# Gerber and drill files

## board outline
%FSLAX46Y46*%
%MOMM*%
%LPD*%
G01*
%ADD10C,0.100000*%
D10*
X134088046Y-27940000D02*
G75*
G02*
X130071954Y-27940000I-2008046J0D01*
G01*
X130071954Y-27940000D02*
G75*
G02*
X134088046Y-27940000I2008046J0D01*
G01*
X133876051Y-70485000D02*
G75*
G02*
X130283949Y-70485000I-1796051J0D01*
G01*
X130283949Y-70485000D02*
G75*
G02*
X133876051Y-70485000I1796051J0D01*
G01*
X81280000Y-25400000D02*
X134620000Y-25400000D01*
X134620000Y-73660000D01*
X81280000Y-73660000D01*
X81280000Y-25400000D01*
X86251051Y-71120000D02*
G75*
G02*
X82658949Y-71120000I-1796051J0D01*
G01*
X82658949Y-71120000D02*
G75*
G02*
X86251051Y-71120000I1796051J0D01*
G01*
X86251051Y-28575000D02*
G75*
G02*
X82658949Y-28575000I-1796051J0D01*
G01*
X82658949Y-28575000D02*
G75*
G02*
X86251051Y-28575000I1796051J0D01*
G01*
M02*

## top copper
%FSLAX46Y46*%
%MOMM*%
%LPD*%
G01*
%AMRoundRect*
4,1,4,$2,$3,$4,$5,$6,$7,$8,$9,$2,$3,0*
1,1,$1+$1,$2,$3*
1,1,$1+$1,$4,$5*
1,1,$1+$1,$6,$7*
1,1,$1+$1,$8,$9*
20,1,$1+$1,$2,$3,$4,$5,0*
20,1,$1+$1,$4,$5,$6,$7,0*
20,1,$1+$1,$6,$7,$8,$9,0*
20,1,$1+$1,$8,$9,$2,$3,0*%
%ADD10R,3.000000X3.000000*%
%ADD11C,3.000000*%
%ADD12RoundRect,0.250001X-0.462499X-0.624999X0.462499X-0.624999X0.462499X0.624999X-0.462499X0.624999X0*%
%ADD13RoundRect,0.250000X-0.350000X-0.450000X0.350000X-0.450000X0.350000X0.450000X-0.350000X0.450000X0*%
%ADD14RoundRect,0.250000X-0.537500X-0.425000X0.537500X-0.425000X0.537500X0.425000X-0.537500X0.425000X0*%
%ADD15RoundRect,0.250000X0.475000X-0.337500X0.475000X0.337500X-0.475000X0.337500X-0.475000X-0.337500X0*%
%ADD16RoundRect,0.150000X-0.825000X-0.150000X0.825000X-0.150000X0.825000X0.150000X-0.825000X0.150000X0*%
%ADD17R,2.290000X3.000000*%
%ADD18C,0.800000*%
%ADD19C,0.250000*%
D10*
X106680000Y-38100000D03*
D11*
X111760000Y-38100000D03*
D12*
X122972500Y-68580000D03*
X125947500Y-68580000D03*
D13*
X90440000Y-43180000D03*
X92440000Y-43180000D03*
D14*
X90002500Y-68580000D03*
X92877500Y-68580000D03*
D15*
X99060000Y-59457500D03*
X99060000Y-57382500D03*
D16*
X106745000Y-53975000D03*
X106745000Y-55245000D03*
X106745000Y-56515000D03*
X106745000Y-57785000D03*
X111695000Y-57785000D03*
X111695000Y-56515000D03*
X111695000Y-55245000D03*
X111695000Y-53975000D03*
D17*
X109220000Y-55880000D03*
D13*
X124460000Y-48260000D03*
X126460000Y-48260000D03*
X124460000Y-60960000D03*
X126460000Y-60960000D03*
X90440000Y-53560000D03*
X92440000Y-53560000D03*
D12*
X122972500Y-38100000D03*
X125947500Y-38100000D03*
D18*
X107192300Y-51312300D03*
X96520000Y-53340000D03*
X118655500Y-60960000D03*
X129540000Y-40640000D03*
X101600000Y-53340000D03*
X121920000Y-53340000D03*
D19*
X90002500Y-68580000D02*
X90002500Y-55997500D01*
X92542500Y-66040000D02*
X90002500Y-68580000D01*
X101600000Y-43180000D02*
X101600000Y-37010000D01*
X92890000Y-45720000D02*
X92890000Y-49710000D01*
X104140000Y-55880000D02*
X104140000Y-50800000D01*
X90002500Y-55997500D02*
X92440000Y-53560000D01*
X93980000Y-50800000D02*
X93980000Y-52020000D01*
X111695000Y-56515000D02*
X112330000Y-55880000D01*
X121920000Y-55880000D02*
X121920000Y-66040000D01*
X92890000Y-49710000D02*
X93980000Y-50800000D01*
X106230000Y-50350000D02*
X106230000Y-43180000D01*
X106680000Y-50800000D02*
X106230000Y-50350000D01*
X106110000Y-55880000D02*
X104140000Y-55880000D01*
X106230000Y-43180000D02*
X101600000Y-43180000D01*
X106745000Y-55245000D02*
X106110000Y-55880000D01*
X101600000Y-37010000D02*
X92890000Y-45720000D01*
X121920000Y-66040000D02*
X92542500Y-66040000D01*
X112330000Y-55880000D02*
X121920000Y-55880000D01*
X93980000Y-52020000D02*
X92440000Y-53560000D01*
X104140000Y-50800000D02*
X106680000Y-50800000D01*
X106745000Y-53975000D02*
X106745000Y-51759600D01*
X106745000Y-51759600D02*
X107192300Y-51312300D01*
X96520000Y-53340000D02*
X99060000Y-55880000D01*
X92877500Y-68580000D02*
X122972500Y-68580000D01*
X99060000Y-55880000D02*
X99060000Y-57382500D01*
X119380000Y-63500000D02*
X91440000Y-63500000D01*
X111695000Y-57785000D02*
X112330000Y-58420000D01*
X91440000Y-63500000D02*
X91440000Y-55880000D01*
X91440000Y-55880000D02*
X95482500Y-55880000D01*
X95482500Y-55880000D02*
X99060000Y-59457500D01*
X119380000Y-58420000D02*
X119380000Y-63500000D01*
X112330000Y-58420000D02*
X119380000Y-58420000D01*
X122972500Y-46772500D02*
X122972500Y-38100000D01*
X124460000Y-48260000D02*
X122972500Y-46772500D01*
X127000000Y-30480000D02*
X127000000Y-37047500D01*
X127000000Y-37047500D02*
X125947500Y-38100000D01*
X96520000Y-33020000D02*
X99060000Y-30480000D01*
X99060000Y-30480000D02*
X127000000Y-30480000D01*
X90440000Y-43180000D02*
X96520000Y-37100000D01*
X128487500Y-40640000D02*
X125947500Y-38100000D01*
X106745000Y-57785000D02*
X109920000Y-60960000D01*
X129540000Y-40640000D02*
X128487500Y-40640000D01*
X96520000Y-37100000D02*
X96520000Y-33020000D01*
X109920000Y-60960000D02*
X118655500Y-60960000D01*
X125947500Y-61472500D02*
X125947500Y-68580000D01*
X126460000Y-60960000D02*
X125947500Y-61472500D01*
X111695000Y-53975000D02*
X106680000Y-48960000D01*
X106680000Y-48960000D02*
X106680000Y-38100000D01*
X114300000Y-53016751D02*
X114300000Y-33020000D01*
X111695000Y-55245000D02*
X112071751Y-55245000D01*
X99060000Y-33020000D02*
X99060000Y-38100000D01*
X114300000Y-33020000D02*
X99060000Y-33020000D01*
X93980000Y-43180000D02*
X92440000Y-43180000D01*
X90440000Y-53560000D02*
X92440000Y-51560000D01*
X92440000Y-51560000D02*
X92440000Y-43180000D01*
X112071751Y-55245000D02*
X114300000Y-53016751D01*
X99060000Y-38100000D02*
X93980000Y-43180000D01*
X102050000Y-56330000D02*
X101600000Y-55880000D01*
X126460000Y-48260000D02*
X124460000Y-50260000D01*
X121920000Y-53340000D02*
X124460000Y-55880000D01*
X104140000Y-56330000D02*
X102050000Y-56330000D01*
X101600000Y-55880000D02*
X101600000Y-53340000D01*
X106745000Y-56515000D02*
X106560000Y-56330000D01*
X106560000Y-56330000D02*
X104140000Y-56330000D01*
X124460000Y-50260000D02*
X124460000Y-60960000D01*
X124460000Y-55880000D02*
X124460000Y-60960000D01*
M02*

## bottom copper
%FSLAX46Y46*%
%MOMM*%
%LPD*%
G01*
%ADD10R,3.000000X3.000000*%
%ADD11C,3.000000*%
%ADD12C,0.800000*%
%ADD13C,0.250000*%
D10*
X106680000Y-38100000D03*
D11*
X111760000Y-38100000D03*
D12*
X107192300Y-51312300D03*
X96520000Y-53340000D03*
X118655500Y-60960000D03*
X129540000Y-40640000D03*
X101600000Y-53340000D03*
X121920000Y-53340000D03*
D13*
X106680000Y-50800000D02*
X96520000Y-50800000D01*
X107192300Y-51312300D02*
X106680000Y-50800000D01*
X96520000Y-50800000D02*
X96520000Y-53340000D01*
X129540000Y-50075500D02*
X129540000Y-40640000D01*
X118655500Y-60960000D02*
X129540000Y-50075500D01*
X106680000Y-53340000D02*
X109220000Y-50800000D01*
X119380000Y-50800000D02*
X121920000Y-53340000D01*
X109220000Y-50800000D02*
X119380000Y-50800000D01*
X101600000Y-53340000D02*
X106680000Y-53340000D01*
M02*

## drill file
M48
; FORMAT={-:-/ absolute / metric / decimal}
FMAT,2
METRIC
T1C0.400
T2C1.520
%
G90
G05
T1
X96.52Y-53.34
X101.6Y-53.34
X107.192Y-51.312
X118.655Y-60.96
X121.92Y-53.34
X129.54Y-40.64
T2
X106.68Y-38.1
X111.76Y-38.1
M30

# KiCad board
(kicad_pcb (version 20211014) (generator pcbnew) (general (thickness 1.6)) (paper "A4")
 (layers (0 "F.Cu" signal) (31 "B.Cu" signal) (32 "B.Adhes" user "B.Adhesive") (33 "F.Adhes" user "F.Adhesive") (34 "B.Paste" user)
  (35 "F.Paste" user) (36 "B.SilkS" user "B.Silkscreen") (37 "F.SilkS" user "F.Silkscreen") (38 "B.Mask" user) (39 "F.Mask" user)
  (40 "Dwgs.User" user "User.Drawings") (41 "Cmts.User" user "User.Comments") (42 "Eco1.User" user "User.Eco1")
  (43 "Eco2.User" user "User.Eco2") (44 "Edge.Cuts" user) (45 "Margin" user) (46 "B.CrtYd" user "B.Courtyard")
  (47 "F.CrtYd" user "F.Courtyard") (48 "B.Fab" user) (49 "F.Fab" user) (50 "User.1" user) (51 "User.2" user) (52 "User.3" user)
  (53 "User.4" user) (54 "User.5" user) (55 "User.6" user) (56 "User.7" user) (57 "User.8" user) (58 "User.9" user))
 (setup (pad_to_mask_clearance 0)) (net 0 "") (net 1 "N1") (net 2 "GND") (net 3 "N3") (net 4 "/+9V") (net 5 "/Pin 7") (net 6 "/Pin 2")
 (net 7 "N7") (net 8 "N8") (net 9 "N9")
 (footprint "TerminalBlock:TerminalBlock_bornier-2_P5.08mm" (layer "F.Cu") (at 106.68 38.1)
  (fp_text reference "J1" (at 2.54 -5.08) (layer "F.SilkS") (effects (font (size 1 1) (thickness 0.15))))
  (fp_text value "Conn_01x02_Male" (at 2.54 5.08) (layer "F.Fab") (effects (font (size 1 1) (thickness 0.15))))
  (pad "1" thru_hole rect (at 0 0) (size 3 3) (drill 1.52) (layers *.Cu *.Mask) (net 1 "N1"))
  (pad "2" thru_hole circle (at 5.08 0) (size 3 3) (drill 1.52) (layers *.Cu *.Mask) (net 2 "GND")))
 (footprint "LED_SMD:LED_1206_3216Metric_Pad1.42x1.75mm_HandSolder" (layer "F.Cu") (at 124.46 68.58)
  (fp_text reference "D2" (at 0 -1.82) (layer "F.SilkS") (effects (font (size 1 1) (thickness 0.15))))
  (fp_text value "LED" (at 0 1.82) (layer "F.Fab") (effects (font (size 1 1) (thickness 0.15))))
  (pad "1" smd roundrect (at -1.4875 0) (size 1.425 1.75) (layers "F.Cu" "F.Paste" "F.Mask") (roundrect_rratio 0.175439) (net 2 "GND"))
  (pad "2" smd roundrect (at 1.4875 0) (size 1.425 1.75) (layers "F.Cu" "F.Paste" "F.Mask") (roundrect_rratio 0.175439) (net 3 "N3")))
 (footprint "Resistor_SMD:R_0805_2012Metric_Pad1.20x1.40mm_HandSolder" (layer "F.Cu") (at 91.44 43.18)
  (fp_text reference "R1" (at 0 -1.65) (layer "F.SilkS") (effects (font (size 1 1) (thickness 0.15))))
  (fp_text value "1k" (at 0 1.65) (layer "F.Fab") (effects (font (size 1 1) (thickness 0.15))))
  (pad "1" smd roundrect (at -1 0) (size 1.2 1.4) (layers "F.Cu" "F.Paste" "F.Mask") (roundrect_rratio 0.208333) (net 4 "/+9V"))
  (pad "2" smd roundrect (at 1 0) (size 1.2 1.4) (layers "F.Cu" "F.Paste" "F.Mask") (roundrect_rratio 0.208333) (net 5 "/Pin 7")))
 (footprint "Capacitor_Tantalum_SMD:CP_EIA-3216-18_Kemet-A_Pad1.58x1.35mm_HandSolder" (layer "F.Cu") (at 91.44 68.58)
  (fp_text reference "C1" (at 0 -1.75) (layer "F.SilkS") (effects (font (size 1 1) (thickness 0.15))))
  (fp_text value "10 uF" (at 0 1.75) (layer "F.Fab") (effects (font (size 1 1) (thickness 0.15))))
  (pad "1" smd roundrect (at -1.4375 0) (size 1.575 1.35) (layers "F.Cu" "F.Paste" "F.Mask") (roundrect_rratio 0.185185) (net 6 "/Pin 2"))
  (pad "2" smd roundrect (at 1.4375 0) (size 1.575 1.35) (layers "F.Cu" "F.Paste" "F.Mask") (roundrect_rratio 0.185185) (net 2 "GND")))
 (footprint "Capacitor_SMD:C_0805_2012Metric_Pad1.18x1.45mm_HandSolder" (layer "F.Cu") (at 99.06 58.42 90)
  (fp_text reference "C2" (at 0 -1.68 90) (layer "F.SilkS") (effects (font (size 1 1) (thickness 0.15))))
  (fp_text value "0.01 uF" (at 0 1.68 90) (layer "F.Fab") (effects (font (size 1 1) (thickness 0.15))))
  (pad "1" smd roundrect (at -1.0375 0 90) (size 1.175 1.45) (layers "F.Cu" "F.Paste" "F.Mask") (roundrect_rratio 0.212766) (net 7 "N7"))
  (pad "2" smd roundrect (at 1.0375 0 90) (size 1.175 1.45) (layers "F.Cu" "F.Paste" "F.Mask") (roundrect_rratio 0.212766) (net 2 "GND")))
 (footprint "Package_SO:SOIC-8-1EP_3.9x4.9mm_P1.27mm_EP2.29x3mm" (layer "F.Cu") (at 109.22 55.88)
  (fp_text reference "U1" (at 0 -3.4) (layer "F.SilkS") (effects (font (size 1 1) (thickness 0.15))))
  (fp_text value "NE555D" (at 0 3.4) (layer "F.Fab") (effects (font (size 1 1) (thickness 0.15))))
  (pad "" smd roundrect (at -0.57 0.75) (size 0.92 1.21) (layers "F.Paste") (roundrect_rratio 0.25))
  (pad "" smd roundrect (at -0.57 -0.75) (size 0.92 1.21) (layers "F.Paste") (roundrect_rratio 0.25))
  (pad "" smd roundrect (at 0.57 -0.75) (size 0.92 1.21) (layers "F.Paste") (roundrect_rratio 0.25))
  (pad "" smd roundrect (at 0.57 0.75) (size 0.92 1.21) (layers "F.Paste") (roundrect_rratio 0.25))
  (pad "1" smd roundrect (at -2.475 -1.905) (size 1.95 0.6) (layers "F.Cu" "F.Paste" "F.Mask") (roundrect_rratio 0.25) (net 2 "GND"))
  (pad "2" smd roundrect (at -2.475 -0.635) (size 1.95 0.6) (layers "F.Cu" "F.Paste" "F.Mask") (roundrect_rratio 0.25) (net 6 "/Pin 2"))
  (pad "3" smd roundrect (at -2.475 0.635) (size 1.95 0.6) (layers "F.Cu" "F.Paste" "F.Mask") (roundrect_rratio 0.25) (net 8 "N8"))
  (pad "4" smd roundrect (at -2.475 1.905) (size 1.95 0.6) (layers "F.Cu" "F.Paste" "F.Mask") (roundrect_rratio 0.25) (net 4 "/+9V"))
  (pad "5" smd roundrect (at 2.475 1.905) (size 1.95 0.6) (layers "F.Cu" "F.Paste" "F.Mask") (roundrect_rratio 0.25) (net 7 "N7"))
  (pad "6" smd roundrect (at 2.475 0.635) (size 1.95 0.6) (layers "F.Cu" "F.Paste" "F.Mask") (roundrect_rratio 0.25) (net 6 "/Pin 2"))
  (pad "7" smd roundrect (at 2.475 -0.635) (size 1.95 0.6) (layers "F.Cu" "F.Paste" "F.Mask") (roundrect_rratio 0.25) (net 5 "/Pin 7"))
  (pad "8" smd roundrect (at 2.475 -1.905) (size 1.95 0.6) (layers "F.Cu" "F.Paste" "F.Mask") (roundrect_rratio 0.25) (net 1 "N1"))
  (pad "9" smd rect (at 0 0) (size 2.29 3) (layers "F.Cu" "F.Mask")))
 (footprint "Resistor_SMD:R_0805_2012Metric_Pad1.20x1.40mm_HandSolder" (layer "F.Cu") (at 125.46 48.26)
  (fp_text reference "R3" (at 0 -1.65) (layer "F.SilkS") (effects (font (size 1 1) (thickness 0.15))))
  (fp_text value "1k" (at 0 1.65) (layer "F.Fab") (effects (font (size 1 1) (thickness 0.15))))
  (pad "1" smd roundrect (at -1 0) (size 1.2 1.4) (layers "F.Cu" "F.Paste" "F.Mask") (roundrect_rratio 0.208333) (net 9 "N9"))
  (pad "2" smd roundrect (at 1 0) (size 1.2 1.4) (layers "F.Cu" "F.Paste" "F.Mask") (roundrect_rratio 0.208333) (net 8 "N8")))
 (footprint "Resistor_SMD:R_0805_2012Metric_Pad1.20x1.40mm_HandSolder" (layer "F.Cu") (at 125.46 60.96)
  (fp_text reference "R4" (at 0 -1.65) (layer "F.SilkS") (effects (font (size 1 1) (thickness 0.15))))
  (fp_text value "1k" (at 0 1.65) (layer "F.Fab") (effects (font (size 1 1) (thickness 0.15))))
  (pad "1" smd roundrect (at -1 0) (size 1.2 1.4) (layers "F.Cu" "F.Paste" "F.Mask") (roundrect_rratio 0.208333) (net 8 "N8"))
  (pad "2" smd roundrect (at 1 0) (size 1.2 1.4) (layers "F.Cu" "F.Paste" "F.Mask") (roundrect_rratio 0.208333) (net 3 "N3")))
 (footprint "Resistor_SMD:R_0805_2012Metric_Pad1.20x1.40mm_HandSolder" (layer "F.Cu") (at 91.44 53.56)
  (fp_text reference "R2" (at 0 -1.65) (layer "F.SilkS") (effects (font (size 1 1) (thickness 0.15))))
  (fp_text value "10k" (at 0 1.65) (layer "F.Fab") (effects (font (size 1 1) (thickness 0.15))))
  (pad "1" smd roundrect (at -1 0) (size 1.2 1.4) (layers "F.Cu" "F.Paste" "F.Mask") (roundrect_rratio 0.208333) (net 5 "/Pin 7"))
  (pad "2" smd roundrect (at 1 0) (size 1.2 1.4) (layers "F.Cu" "F.Paste" "F.Mask") (roundrect_rratio 0.208333) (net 6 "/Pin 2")))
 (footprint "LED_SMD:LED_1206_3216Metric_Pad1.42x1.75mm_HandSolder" (layer "F.Cu") (at 124.46 38.1)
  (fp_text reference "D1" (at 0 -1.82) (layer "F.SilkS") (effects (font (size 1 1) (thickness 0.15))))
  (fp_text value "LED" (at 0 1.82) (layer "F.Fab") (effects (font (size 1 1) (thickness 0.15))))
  (pad "1" smd roundrect (at -1.4875 0) (size 1.425 1.75) (layers "F.Cu" "F.Paste" "F.Mask") (roundrect_rratio 0.175439) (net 9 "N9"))
  (pad "2" smd roundrect (at 1.4875 0) (size 1.425 1.75) (layers "F.Cu" "F.Paste" "F.Mask") (roundrect_rratio 0.175439) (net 4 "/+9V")))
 (gr_circle (center 132.08 27.94) (end 130.175 28.575) (layer "Edge.Cuts") (width 0.1) (fill none))
 (gr_circle (center 132.08 70.485) (end 130.81 69.215) (layer "Edge.Cuts") (width 0.1) (fill none))
 (gr_rect (start 81.28 25.4) (end 134.62 73.66) (layer "Edge.Cuts") (width 0.1) (fill none))
 (gr_circle (center 84.455 71.12) (end 85.725 69.85) (layer "Edge.Cuts") (width 0.1) (fill none))
 (gr_circle (center 84.455 28.575) (end 85.725 29.845) (layer "Edge.Cuts") (width 0.1) (fill none))
 (segment (start 90.0025 68.58) (end 90.0025 55.9975) (width 0.25) (layer "F.Cu") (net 6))
 (segment (start 92.5425 66.04) (end 90.0025 68.58) (width 0.25) (layer "F.Cu") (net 6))
 (segment (start 101.6 43.18) (end 101.6 37.01) (width 0.25) (layer "F.Cu") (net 6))
 (segment (start 92.89 45.72) (end 92.89 49.71) (width 0.25) (layer "F.Cu") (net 6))
 (segment (start 104.14 55.88) (end 104.14 50.8) (width 0.25) (layer "F.Cu") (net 6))
 (segment (start 90.0025 55.9975) (end 92.44 53.56) (width 0.25) (layer "F.Cu") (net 6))
 (segment (start 93.98 50.8) (end 93.98 52.02) (width 0.25) (layer "F.Cu") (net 6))
 (segment (start 111.695 56.515) (end 112.33 55.88) (width 0.25) (layer "F.Cu") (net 6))
 (segment (start 121.92 55.88) (end 121.92 66.04) (width 0.25) (layer "F.Cu") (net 6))
 (segment (start 92.89 49.71) (end 93.98 50.8) (width 0.25) (layer "F.Cu") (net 6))
 (segment (start 106.23 50.35) (end 106.23 43.18) (width 0.25) (layer "F.Cu") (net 6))
 (segment (start 106.68 50.8) (end 106.23 50.35) (width 0.25) (layer "F.Cu") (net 6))
 (segment (start 106.11 55.88) (end 104.14 55.88) (width 0.25) (layer "F.Cu") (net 6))
 (segment (start 106.23 43.18) (end 101.6 43.18) (width 0.25) (layer "F.Cu") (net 6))
 (segment (start 106.745 55.245) (end 106.11 55.88) (width 0.25) (layer "F.Cu") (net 6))
 (segment (start 101.6 37.01) (end 92.89 45.72) (width 0.25) (layer "F.Cu") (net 6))
 (segment (start 121.92 66.04) (end 92.5425 66.04) (width 0.25) (layer "F.Cu") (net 6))
 (segment (start 112.33 55.88) (end 121.92 55.88) (width 0.25) (layer "F.Cu") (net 6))
 (segment (start 93.98 52.02) (end 92.44 53.56) (width 0.25) (layer "F.Cu") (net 6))
 (segment (start 104.14 50.8) (end 106.68 50.8) (width 0.25) (layer "F.Cu") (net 6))
 (segment (start 106.745 53.975) (end 106.745 51.7596) (width 0.25) (layer "F.Cu") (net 2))
 (segment (start 106.745 51.7596) (end 107.1923 51.3123) (width 0.25) (layer "F.Cu") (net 2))
 (segment (start 96.52 53.34) (end 99.06 55.88) (width 0.25) (layer "F.Cu") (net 2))
 (segment (start 92.8775 68.58) (end 122.9725 68.58) (width 0.25) (layer "F.Cu") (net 2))
 (segment (start 99.06 55.88) (end 99.06 57.3825) (width 0.25) (layer "F.Cu") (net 2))
 (via (at 107.1923 51.3123) (size 0.8) (drill 0.4) (layers "F.Cu" "B.Cu") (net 2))
 (via (at 96.52 53.34) (size 0.8) (drill 0.4) (layers "F.Cu" "B.Cu") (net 2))
 (segment (start 106.68 50.8) (end 96.52 50.8) (width 0.25) (layer "B.Cu") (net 2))
 (segment (start 107.1923 51.3123) (end 106.68 50.8) (width 0.25) (layer "B.Cu") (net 2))
 (segment (start 96.52 50.8) (end 96.52 53.34) (width 0.25) (layer "B.Cu") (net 2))
 (segment (start 119.38 63.5) (end 91.44 63.5) (width 0.25) (layer "F.Cu") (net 7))
 (segment (start 111.695 57.785) (end 112.33 58.42) (width 0.25) (layer "F.Cu") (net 7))
 (segment (start 91.44 63.5) (end 91.44 55.88) (width 0.25) (layer "F.Cu") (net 7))
 (segment (start 91.44 55.88) (end 95.4825 55.88) (width 0.25) (layer "F.Cu") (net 7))
 (segment (start 95.4825 55.88) (end 99.06 59.4575) (width 0.25) (layer "F.Cu") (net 7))
 (segment (start 119.38 58.42) (end 119.38 63.5) (width 0.25) (layer "F.Cu") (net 7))
 (segment (start 112.33 58.42) (end 119.38 58.42) (width 0.25) (layer "F.Cu") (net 7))
 (segment (start 122.9725 46.7725) (end 122.9725 38.1) (width 0.25) (layer "F.Cu") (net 9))
 (segment (start 124.46 48.26) (end 122.9725 46.7725) (width 0.25) (layer "F.Cu") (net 9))
 (segment (start 127 30.48) (end 127 37.0475) (width 0.25) (layer "F.Cu") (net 4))
 (segment (start 127 37.0475) (end 125.9475 38.1) (width 0.25) (layer "F.Cu") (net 4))
 (segment (start 96.52 33.02) (end 99.06 30.48) (width 0.25) (layer "F.Cu") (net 4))
 (segment (start 99.06 30.48) (end 127 30.48) (width 0.25) (layer "F.Cu") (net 4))
 (segment (start 90.44 43.18) (end 96.52 37.1) (width 0.25) (layer "F.Cu") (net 4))
 (segment (start 128.4875 40.64) (end 125.9475 38.1) (width 0.25) (layer "F.Cu") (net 4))
 (segment (start 106.745 57.785) (end 109.92 60.96) (width 0.25) (layer "F.Cu") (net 4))
 (segment (start 129.54 40.64) (end 128.4875 40.64) (width 0.25) (layer "F.Cu") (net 4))
 (segment (start 96.52 37.1) (end 96.52 33.02) (width 0.25) (layer "F.Cu") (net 4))
 (segment (start 109.92 60.96) (end 118.6555 60.96) (width 0.25) (layer "F.Cu") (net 4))
 (via (at 118.6555 60.96) (size 0.8) (drill 0.4) (layers "F.Cu" "B.Cu") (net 4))
 (via (at 129.54 40.64) (size 0.8) (drill 0.4) (layers "F.Cu" "B.Cu") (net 4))
 (segment (start 129.54 50.0755) (end 129.54 40.64) (width 0.25) (layer "B.Cu") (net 4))
 (segment (start 118.6555 60.96) (end 129.54 50.0755) (width 0.25) (layer "B.Cu") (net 4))
 (segment (start 125.9475 61.4725) (end 125.9475 68.58) (width 0.25) (layer "F.Cu") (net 3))
 (segment (start 126.46 60.96) (end 125.9475 61.4725) (width 0.25) (layer "F.Cu") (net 3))
 (segment (start 111.695 53.975) (end 106.68 48.96) (width 0.25) (layer "F.Cu") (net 1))
 (segment (start 106.68 48.96) (end 106.68 38.1) (width 0.25) (layer "F.Cu") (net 1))
 (segment (start 114.3 53.016751) (end 114.3 33.02) (width 0.25) (layer "F.Cu") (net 5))
 (segment (start 111.695 55.245) (end 112.071751 55.245) (width 0.25) (layer "F.Cu") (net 5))
 (segment (start 99.06 33.02) (end 99.06 38.1) (width 0.25) (layer "F.Cu") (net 5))
 (segment (start 114.3 33.02) (end 99.06 33.02) (width 0.25) (layer "F.Cu") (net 5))
 (segment (start 93.98 43.18) (end 92.44 43.18) (width 0.25) (layer "F.Cu") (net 5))
 (segment (start 90.44 53.56) (end 92.44 51.56) (width 0.25) (layer "F.Cu") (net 5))
 (segment (start 92.44 51.56) (end 92.44 43.18) (width 0.25) (layer "F.Cu") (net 5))
 (segment (start 112.071751 55.245) (end 114.3 53.016751) (width 0.25) (layer "F.Cu") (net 5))
 (segment (start 99.06 38.1) (end 93.98 43.18) (width 0.25) (layer "F.Cu") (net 5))
 (segment (start 102.05 56.33) (end 101.6 55.88) (width 0.25) (layer "F.Cu") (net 8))
 (segment (start 126.46 48.26) (end 124.46 50.26) (width 0.25) (layer "F.Cu") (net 8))
 (segment (start 121.92 53.34) (end 124.46 55.88) (width 0.25) (layer "F.Cu") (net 8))
 (segment (start 104.14 56.33) (end 102.05 56.33) (width 0.25) (layer "F.Cu") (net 8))
 (segment (start 101.6 55.88) (end 101.6 53.34) (width 0.25) (layer "F.Cu") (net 8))
 (segment (start 106.745 56.515) (end 106.56 56.33) (width 0.25) (layer "F.Cu") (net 8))
 (segment (start 106.56 56.33) (end 104.14 56.33) (width 0.25) (layer "F.Cu") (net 8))
 (segment (start 124.46 50.26) (end 124.46 60.96) (width 0.25) (layer "F.Cu") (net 8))
 (segment (start 124.46 55.88) (end 124.46 60.96) (width 0.25) (layer "F.Cu") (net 8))
 (via (at 101.6 53.34) (size 0.8) (drill 0.4) (layers "F.Cu" "B.Cu") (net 8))
 (via (at 121.92 53.34) (size 0.8) (drill 0.4) (layers "F.Cu" "B.Cu") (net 8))
 (segment (start 106.68 53.34) (end 109.22 50.8) (width 0.25) (layer "B.Cu") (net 8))
 (segment (start 119.38 50.8) (end 121.92 53.34) (width 0.25) (layer "B.Cu") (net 8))
 (segment (start 109.22 50.8) (end 119.38 50.8) (width 0.25) (layer "B.Cu") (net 8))
 (segment (start 101.6 53.34) (end 106.68 53.34) (width 0.25) (layer "B.Cu") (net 8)))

